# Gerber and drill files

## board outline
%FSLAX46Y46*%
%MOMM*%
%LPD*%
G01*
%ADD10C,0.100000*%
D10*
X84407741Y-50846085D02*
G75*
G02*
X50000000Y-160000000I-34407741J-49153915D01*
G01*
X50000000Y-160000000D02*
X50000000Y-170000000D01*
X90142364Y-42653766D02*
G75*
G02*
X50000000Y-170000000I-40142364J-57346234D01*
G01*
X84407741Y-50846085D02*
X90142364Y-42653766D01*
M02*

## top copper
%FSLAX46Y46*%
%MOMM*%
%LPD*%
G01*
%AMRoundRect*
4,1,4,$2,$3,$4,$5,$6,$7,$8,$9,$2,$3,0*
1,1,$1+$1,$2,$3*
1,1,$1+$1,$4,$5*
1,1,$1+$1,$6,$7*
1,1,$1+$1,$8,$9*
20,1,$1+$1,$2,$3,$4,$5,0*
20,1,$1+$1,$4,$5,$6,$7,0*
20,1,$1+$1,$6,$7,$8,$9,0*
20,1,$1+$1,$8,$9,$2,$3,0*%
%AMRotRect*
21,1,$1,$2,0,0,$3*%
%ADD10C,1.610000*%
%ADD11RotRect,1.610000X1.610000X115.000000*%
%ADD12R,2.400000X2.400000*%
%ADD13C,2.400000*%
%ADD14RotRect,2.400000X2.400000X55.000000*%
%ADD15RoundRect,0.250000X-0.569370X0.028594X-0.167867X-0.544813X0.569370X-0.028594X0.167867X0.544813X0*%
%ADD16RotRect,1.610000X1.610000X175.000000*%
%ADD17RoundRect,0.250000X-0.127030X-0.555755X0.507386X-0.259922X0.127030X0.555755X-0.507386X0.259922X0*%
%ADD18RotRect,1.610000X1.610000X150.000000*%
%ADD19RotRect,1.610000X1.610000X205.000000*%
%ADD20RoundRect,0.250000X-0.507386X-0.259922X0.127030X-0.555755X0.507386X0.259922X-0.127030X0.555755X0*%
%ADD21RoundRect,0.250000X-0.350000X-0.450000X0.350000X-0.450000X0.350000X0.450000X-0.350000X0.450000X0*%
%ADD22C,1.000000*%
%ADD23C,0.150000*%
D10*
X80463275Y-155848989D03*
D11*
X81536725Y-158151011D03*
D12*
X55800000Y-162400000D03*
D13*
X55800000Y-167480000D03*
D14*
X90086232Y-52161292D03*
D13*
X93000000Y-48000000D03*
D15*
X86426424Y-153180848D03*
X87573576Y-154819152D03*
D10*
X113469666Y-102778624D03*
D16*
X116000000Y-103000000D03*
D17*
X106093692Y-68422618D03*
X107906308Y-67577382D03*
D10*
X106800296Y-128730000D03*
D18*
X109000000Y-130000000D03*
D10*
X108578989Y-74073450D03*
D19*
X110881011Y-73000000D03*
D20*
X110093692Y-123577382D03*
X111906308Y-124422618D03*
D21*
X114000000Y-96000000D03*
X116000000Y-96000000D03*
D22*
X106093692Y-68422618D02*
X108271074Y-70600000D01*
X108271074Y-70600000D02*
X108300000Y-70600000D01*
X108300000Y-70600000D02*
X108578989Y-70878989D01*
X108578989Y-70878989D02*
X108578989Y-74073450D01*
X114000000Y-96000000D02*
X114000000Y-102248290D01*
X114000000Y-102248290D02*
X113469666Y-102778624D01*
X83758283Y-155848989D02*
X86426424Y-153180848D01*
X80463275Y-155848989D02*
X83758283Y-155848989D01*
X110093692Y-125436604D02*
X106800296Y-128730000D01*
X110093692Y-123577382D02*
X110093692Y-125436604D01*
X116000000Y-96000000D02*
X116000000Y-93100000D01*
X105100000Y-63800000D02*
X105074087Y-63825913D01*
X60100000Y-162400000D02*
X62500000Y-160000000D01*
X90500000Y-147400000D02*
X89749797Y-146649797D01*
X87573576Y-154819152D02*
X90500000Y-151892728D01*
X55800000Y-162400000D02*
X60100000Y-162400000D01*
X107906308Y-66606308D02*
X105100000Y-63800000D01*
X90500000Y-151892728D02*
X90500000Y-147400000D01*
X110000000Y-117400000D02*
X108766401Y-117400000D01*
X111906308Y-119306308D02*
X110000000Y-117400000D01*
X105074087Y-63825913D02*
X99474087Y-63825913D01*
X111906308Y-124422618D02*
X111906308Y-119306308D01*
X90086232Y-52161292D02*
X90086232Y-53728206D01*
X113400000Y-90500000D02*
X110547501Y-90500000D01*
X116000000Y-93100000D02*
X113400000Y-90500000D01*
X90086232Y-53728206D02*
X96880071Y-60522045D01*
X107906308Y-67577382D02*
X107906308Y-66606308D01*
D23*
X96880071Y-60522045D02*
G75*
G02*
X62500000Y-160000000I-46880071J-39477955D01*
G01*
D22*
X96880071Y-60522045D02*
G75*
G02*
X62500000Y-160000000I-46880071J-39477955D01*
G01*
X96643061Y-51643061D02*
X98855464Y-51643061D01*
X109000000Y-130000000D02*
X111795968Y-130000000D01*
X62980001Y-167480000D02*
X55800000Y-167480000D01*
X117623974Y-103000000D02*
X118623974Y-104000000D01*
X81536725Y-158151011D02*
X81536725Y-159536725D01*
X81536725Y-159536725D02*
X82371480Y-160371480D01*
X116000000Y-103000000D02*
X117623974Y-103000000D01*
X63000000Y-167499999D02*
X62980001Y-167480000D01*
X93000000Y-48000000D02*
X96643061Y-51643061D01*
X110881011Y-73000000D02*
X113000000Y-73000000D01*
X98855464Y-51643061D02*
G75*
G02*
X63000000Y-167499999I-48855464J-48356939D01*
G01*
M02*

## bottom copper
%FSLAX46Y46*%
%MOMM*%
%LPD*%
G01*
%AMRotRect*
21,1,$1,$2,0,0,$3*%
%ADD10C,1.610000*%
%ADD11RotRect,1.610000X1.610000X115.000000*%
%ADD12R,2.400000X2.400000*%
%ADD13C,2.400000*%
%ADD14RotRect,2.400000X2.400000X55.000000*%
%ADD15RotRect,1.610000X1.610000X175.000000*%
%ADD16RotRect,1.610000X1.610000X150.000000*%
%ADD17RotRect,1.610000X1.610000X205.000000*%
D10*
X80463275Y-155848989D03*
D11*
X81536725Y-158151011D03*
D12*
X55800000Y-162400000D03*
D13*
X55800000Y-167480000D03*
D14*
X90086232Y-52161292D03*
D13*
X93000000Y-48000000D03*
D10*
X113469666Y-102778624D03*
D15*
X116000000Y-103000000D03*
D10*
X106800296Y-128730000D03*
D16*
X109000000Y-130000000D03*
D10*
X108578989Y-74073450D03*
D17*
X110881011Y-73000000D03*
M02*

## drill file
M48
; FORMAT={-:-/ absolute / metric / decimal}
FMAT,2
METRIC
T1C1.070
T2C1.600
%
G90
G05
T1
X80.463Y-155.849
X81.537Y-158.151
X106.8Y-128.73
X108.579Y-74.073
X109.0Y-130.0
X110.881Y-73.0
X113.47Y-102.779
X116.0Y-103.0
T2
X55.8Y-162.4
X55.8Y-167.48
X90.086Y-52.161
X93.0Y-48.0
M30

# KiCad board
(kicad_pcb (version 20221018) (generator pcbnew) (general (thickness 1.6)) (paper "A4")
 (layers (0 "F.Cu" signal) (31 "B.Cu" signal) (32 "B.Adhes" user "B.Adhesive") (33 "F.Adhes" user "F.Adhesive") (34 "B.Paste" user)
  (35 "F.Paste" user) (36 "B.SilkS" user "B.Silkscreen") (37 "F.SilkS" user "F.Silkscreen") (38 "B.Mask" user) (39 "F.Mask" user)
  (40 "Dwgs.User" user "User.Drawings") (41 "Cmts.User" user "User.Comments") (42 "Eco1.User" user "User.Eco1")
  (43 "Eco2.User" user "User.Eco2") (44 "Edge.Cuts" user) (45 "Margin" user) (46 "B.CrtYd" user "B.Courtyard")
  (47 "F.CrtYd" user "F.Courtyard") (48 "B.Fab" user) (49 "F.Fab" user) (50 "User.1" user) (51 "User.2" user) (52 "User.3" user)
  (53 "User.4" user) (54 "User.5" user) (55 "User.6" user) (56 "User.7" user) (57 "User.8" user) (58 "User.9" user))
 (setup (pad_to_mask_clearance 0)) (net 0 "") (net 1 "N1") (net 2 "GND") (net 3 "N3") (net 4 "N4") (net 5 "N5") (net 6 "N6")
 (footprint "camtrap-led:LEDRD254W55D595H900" (layer "F.Cu") (at 81 157 115)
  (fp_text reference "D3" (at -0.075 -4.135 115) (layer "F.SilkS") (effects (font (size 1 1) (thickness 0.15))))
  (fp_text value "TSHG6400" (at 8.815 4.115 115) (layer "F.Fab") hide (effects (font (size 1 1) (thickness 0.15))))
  (pad "A" thru_hole circle (at 1.27 0 115) (size 1.61 1.61) (drill 1.07) (layers "*.Cu" "*.Mask") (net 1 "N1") (solder_mask_margin 0.102))
  (pad "C" thru_hole rect (at -1.27 0 115) (size 1.61 1.61) (drill 1.07) (layers "*.Cu" "*.Mask") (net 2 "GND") (solder_mask_margin 0.102)))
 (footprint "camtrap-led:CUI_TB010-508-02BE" (layer "F.Cu") (at 55.8 162.4 -90)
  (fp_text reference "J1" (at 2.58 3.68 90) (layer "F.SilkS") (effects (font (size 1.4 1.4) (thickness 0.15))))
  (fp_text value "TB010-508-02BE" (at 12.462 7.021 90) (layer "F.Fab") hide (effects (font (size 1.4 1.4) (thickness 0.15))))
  (pad "1" thru_hole rect (at 0 0 270) (size 2.4 2.4) (drill 1.6) (layers "*.Cu" "*.Mask") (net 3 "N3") (solder_mask_margin 0.102))
  (pad "2" thru_hole circle (at 5.08 0 270) (size 2.4 2.4) (drill 1.6) (layers "*.Cu" "*.Mask") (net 2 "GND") (solder_mask_margin 0.102)))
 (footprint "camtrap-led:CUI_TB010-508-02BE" (layer "F.Cu") (at 90.086232 52.161292 55)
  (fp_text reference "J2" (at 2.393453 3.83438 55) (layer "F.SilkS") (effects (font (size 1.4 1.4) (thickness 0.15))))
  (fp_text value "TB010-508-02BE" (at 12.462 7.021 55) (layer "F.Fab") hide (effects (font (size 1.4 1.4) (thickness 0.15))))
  (pad "1" thru_hole rect (at 0 0 55) (size 2.4 2.4) (drill 1.6) (layers "*.Cu" "*.Mask") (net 3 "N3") (solder_mask_margin 0.102))
  (pad "2" thru_hole circle (at 5.08 0 55) (size 2.4 2.4) (drill 1.6) (layers "*.Cu" "*.Mask") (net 2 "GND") (solder_mask_margin 0.102)))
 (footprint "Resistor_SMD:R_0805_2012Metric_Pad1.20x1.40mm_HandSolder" (layer "F.Cu") (at 87 154 -55)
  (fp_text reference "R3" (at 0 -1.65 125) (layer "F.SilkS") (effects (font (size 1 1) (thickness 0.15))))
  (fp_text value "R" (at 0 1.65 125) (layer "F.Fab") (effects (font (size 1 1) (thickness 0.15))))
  (pad "1" smd roundrect (at -1 0 305) (size 1.2 1.4) (layers "F.Cu" "F.Paste" "F.Mask") (roundrect_rratio 0.2083333333) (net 1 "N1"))
  (pad "2" smd roundrect (at 1 0 305) (size 1.2 1.4) (layers "F.Cu" "F.Paste" "F.Mask") (roundrect_rratio 0.2083333333) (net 3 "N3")))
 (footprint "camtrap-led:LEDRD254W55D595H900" (layer "F.Cu") (at 114.734833 102.889312 175)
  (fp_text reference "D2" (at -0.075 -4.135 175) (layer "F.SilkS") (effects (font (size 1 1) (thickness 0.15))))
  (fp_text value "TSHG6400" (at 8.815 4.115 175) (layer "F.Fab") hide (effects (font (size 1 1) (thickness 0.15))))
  (pad "A" thru_hole circle (at 1.27 0 175) (size 1.61 1.61) (drill 1.07) (layers "*.Cu" "*.Mask") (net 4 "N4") (solder_mask_margin 0.102))
  (pad "C" thru_hole rect (at -1.27 0 175) (size 1.61 1.61) (drill 1.07) (layers "*.Cu" "*.Mask") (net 2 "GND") (solder_mask_margin 0.102)))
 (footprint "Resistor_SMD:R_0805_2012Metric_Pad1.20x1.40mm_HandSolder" (layer "F.Cu") (at 107 68 25)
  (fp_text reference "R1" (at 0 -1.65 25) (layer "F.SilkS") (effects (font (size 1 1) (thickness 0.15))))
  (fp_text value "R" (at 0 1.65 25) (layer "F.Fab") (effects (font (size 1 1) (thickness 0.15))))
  (pad "1" smd roundrect (at -1 0 25) (size 1.2 1.4) (layers "F.Cu" "F.Paste" "F.Mask") (roundrect_rratio 0.2083333333) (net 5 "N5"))
  (pad "2" smd roundrect (at 1 0 25) (size 1.2 1.4) (layers "F.Cu" "F.Paste" "F.Mask") (roundrect_rratio 0.2083333333) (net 3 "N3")))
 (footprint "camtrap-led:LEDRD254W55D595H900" (layer "F.Cu") (at 107.900148 129.365 150)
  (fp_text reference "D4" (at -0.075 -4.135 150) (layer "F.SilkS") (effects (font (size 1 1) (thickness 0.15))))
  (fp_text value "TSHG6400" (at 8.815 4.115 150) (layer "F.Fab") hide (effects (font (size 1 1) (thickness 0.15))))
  (pad "A" thru_hole circle (at 1.27 0 150) (size 1.61 1.61) (drill 1.07) (layers "*.Cu" "*.Mask") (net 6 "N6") (solder_mask_margin 0.102))
  (pad "C" thru_hole rect (at -1.27 0 150) (size 1.61 1.61) (drill 1.07) (layers "*.Cu" "*.Mask") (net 2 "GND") (solder_mask_margin 0.102)))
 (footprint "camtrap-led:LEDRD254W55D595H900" (layer "F.Cu") (at 109.73 73.536725 -155)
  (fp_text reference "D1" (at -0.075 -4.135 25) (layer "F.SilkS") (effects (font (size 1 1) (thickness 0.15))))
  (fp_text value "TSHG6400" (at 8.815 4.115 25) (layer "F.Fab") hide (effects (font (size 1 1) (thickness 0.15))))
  (pad "A" thru_hole circle (at 1.27 0 205) (size 1.61 1.61) (drill 1.07) (layers "*.Cu" "*.Mask") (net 5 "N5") (solder_mask_margin 0.102))
  (pad "C" thru_hole rect (at -1.27 0 205) (size 1.61 1.61) (drill 1.07) (layers "*.Cu" "*.Mask") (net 2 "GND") (solder_mask_margin 0.102)))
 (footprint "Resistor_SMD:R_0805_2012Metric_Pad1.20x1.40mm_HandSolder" (layer "F.Cu") (at 111 124 -25)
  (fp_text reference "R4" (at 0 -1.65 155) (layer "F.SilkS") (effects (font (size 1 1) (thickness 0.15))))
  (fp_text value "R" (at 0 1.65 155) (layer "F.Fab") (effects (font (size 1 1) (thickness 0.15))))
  (pad "1" smd roundrect (at -1 0 335) (size 1.2 1.4) (layers "F.Cu" "F.Paste" "F.Mask") (roundrect_rratio 0.2083333333) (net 6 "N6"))
  (pad "2" smd roundrect (at 1 0 335) (size 1.2 1.4) (layers "F.Cu" "F.Paste" "F.Mask") (roundrect_rratio 0.2083333333) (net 3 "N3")))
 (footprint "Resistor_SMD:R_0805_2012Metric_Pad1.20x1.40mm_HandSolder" (layer "F.Cu") (at 115 96)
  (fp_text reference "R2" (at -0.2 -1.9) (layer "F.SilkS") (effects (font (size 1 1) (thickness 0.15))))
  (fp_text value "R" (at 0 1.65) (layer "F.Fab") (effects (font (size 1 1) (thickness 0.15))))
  (pad "1" smd roundrect (at -1 0) (size 1.2 1.4) (layers "F.Cu" "F.Paste" "F.Mask") (roundrect_rratio 0.2083333333) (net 4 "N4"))
  (pad "2" smd roundrect (at 1 0) (size 1.2 1.4) (layers "F.Cu" "F.Paste" "F.Mask") (roundrect_rratio 0.2083333333) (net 3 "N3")))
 (gr_arc (start 84.407741 50.846085) (mid 107.224273 118.038363) (end 50 160) (stroke (width 0.1) (type default)) (layer "Edge.Cuts"))
 (gr_line (start 50 160) (end 50 170) (stroke (width 0.1) (type default)) (layer "Edge.Cuts"))
 (gr_arc (start 90.142364 42.653766) (mid 116.761652 121.044757) (end 50 170) (stroke (width 0.1) (type default)) (layer "Edge.Cuts"))
 (gr_line (start 84.407741 50.846085) (end 90.142364 42.653766) (stroke (width 0.1) (type default)) (layer "Edge.Cuts"))
 (segment (start 106.093692 68.422618) (end 108.271074 70.6) (width 1) (layer "F.Cu") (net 5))
 (segment (start 108.271074 70.6) (end 108.3 70.6) (width 1) (layer "F.Cu") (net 5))
 (segment (start 108.3 70.6) (end 108.578989 70.878989) (width 1) (layer "F.Cu") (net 5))
 (segment (start 108.578989 70.878989) (end 108.578989 74.07345) (width 1) (layer "F.Cu") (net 5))
 (segment (start 114 96) (end 114 102.24829) (width 1) (layer "F.Cu") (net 4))
 (segment (start 114 102.24829) (end 113.469666 102.778624) (width 1) (layer "F.Cu") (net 4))
 (segment (start 83.758283 155.848989) (end 86.426424 153.180848) (width 1) (layer "F.Cu") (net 1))
 (segment (start 80.463275 155.848989) (end 83.758283 155.848989) (width 1) (layer "F.Cu") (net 1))
 (segment (start 110.093692 125.436604) (end 106.800296 128.73) (width 1) (layer "F.Cu") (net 6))
 (segment (start 110.093692 123.577382) (end 110.093692 125.436604) (width 1) (layer "F.Cu") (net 6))
 (segment (start 116 96) (end 116 93.1) (width 1) (layer "F.Cu") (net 3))
 (segment (start 105.1 63.8) (end 105.074087 63.825913) (width 1) (layer "F.Cu") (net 3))
 (segment (start 60.1 162.4) (end 62.5 160) (width 1) (layer "F.Cu") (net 3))
 (segment (start 90.5 147.4) (end 89.749797 146.649797) (width 1) (layer "F.Cu") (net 3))
 (segment (start 87.573576 154.819152) (end 90.5 151.892728) (width 1) (layer "F.Cu") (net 3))
 (segment (start 55.8 162.4) (end 60.1 162.4) (width 1) (layer "F.Cu") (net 3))
 (segment (start 107.906308 66.606308) (end 105.1 63.8) (width 1) (layer "F.Cu") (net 3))
 (segment (start 90.5 151.892728) (end 90.5 147.4) (width 1) (layer "F.Cu") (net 3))
 (segment (start 110 117.4) (end 108.766401 117.4) (width 1) (layer "F.Cu") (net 3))
 (segment (start 111.906308 119.306308) (end 110 117.4) (width 1) (layer "F.Cu") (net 3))
 (segment (start 105.074087 63.825913) (end 99.474087 63.825913) (width 1) (layer "F.Cu") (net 3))
 (segment (start 111.906308 124.422618) (end 111.906308 119.306308) (width 1) (layer "F.Cu") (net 3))
 (segment (start 90.086232 52.161292) (end 90.086232 53.728206) (width 1) (layer "F.Cu") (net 3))
 (segment (start 113.4 90.5) (end 110.547501 90.5) (width 1) (layer "F.Cu") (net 3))
 (segment (start 116 93.1) (end 113.4 90.5) (width 1) (layer "F.Cu") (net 3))
 (segment (start 90.086232 53.728206) (end 96.880071 60.522045) (width 1) (layer "F.Cu") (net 3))
 (segment (start 107.906308 67.577382) (end 107.906308 66.606308) (width 1) (layer "F.Cu") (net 3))
 (arc (start 96.880071 60.522045) (mid 107.926368 120.019638) (end 62.5 160) (width 0.15) (layer "F.Cu") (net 3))
 (arc (start 96.880071 60.522045) (mid 107.926368 120.019638) (end 62.5 160) (width 1) (layer "F.Cu") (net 3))
 (segment (start 96.643061 51.643061) (end 98.855464 51.643061) (width 1) (layer "F.Cu") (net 2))
 (segment (start 109 130) (end 111.795968 130) (width 1) (layer "F.Cu") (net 2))
 (segment (start 62.980001 167.48) (end 55.8 167.48) (width 1) (layer "F.Cu") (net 2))
 (segment (start 117.623974 103) (end 118.623974 104) (width 1) (layer "F.Cu") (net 2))
 (segment (start 81.536725 158.151011) (end 81.536725 159.536725) (width 1) (layer "F.Cu") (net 2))
 (segment (start 81.536725 159.536725) (end 82.37148 160.37148) (width 1) (layer "F.Cu") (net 2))
 (segment (start 116 103) (end 117.623974 103) (width 1) (layer "F.Cu") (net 2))
 (segment (start 63 167.499999) (end 62.980001 167.48) (width 1) (layer "F.Cu") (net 2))
 (segment (start 93 48) (end 96.643061 51.643061) (width 1) (layer "F.Cu") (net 2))
 (segment (start 110.881011 73) (end 113 73) (width 1) (layer "F.Cu") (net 2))
 (arc (start 98.855464 51.643061) (mid 115.667588 120.322838) (end 63 167.499999) (width 1) (layer "F.Cu") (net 2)))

